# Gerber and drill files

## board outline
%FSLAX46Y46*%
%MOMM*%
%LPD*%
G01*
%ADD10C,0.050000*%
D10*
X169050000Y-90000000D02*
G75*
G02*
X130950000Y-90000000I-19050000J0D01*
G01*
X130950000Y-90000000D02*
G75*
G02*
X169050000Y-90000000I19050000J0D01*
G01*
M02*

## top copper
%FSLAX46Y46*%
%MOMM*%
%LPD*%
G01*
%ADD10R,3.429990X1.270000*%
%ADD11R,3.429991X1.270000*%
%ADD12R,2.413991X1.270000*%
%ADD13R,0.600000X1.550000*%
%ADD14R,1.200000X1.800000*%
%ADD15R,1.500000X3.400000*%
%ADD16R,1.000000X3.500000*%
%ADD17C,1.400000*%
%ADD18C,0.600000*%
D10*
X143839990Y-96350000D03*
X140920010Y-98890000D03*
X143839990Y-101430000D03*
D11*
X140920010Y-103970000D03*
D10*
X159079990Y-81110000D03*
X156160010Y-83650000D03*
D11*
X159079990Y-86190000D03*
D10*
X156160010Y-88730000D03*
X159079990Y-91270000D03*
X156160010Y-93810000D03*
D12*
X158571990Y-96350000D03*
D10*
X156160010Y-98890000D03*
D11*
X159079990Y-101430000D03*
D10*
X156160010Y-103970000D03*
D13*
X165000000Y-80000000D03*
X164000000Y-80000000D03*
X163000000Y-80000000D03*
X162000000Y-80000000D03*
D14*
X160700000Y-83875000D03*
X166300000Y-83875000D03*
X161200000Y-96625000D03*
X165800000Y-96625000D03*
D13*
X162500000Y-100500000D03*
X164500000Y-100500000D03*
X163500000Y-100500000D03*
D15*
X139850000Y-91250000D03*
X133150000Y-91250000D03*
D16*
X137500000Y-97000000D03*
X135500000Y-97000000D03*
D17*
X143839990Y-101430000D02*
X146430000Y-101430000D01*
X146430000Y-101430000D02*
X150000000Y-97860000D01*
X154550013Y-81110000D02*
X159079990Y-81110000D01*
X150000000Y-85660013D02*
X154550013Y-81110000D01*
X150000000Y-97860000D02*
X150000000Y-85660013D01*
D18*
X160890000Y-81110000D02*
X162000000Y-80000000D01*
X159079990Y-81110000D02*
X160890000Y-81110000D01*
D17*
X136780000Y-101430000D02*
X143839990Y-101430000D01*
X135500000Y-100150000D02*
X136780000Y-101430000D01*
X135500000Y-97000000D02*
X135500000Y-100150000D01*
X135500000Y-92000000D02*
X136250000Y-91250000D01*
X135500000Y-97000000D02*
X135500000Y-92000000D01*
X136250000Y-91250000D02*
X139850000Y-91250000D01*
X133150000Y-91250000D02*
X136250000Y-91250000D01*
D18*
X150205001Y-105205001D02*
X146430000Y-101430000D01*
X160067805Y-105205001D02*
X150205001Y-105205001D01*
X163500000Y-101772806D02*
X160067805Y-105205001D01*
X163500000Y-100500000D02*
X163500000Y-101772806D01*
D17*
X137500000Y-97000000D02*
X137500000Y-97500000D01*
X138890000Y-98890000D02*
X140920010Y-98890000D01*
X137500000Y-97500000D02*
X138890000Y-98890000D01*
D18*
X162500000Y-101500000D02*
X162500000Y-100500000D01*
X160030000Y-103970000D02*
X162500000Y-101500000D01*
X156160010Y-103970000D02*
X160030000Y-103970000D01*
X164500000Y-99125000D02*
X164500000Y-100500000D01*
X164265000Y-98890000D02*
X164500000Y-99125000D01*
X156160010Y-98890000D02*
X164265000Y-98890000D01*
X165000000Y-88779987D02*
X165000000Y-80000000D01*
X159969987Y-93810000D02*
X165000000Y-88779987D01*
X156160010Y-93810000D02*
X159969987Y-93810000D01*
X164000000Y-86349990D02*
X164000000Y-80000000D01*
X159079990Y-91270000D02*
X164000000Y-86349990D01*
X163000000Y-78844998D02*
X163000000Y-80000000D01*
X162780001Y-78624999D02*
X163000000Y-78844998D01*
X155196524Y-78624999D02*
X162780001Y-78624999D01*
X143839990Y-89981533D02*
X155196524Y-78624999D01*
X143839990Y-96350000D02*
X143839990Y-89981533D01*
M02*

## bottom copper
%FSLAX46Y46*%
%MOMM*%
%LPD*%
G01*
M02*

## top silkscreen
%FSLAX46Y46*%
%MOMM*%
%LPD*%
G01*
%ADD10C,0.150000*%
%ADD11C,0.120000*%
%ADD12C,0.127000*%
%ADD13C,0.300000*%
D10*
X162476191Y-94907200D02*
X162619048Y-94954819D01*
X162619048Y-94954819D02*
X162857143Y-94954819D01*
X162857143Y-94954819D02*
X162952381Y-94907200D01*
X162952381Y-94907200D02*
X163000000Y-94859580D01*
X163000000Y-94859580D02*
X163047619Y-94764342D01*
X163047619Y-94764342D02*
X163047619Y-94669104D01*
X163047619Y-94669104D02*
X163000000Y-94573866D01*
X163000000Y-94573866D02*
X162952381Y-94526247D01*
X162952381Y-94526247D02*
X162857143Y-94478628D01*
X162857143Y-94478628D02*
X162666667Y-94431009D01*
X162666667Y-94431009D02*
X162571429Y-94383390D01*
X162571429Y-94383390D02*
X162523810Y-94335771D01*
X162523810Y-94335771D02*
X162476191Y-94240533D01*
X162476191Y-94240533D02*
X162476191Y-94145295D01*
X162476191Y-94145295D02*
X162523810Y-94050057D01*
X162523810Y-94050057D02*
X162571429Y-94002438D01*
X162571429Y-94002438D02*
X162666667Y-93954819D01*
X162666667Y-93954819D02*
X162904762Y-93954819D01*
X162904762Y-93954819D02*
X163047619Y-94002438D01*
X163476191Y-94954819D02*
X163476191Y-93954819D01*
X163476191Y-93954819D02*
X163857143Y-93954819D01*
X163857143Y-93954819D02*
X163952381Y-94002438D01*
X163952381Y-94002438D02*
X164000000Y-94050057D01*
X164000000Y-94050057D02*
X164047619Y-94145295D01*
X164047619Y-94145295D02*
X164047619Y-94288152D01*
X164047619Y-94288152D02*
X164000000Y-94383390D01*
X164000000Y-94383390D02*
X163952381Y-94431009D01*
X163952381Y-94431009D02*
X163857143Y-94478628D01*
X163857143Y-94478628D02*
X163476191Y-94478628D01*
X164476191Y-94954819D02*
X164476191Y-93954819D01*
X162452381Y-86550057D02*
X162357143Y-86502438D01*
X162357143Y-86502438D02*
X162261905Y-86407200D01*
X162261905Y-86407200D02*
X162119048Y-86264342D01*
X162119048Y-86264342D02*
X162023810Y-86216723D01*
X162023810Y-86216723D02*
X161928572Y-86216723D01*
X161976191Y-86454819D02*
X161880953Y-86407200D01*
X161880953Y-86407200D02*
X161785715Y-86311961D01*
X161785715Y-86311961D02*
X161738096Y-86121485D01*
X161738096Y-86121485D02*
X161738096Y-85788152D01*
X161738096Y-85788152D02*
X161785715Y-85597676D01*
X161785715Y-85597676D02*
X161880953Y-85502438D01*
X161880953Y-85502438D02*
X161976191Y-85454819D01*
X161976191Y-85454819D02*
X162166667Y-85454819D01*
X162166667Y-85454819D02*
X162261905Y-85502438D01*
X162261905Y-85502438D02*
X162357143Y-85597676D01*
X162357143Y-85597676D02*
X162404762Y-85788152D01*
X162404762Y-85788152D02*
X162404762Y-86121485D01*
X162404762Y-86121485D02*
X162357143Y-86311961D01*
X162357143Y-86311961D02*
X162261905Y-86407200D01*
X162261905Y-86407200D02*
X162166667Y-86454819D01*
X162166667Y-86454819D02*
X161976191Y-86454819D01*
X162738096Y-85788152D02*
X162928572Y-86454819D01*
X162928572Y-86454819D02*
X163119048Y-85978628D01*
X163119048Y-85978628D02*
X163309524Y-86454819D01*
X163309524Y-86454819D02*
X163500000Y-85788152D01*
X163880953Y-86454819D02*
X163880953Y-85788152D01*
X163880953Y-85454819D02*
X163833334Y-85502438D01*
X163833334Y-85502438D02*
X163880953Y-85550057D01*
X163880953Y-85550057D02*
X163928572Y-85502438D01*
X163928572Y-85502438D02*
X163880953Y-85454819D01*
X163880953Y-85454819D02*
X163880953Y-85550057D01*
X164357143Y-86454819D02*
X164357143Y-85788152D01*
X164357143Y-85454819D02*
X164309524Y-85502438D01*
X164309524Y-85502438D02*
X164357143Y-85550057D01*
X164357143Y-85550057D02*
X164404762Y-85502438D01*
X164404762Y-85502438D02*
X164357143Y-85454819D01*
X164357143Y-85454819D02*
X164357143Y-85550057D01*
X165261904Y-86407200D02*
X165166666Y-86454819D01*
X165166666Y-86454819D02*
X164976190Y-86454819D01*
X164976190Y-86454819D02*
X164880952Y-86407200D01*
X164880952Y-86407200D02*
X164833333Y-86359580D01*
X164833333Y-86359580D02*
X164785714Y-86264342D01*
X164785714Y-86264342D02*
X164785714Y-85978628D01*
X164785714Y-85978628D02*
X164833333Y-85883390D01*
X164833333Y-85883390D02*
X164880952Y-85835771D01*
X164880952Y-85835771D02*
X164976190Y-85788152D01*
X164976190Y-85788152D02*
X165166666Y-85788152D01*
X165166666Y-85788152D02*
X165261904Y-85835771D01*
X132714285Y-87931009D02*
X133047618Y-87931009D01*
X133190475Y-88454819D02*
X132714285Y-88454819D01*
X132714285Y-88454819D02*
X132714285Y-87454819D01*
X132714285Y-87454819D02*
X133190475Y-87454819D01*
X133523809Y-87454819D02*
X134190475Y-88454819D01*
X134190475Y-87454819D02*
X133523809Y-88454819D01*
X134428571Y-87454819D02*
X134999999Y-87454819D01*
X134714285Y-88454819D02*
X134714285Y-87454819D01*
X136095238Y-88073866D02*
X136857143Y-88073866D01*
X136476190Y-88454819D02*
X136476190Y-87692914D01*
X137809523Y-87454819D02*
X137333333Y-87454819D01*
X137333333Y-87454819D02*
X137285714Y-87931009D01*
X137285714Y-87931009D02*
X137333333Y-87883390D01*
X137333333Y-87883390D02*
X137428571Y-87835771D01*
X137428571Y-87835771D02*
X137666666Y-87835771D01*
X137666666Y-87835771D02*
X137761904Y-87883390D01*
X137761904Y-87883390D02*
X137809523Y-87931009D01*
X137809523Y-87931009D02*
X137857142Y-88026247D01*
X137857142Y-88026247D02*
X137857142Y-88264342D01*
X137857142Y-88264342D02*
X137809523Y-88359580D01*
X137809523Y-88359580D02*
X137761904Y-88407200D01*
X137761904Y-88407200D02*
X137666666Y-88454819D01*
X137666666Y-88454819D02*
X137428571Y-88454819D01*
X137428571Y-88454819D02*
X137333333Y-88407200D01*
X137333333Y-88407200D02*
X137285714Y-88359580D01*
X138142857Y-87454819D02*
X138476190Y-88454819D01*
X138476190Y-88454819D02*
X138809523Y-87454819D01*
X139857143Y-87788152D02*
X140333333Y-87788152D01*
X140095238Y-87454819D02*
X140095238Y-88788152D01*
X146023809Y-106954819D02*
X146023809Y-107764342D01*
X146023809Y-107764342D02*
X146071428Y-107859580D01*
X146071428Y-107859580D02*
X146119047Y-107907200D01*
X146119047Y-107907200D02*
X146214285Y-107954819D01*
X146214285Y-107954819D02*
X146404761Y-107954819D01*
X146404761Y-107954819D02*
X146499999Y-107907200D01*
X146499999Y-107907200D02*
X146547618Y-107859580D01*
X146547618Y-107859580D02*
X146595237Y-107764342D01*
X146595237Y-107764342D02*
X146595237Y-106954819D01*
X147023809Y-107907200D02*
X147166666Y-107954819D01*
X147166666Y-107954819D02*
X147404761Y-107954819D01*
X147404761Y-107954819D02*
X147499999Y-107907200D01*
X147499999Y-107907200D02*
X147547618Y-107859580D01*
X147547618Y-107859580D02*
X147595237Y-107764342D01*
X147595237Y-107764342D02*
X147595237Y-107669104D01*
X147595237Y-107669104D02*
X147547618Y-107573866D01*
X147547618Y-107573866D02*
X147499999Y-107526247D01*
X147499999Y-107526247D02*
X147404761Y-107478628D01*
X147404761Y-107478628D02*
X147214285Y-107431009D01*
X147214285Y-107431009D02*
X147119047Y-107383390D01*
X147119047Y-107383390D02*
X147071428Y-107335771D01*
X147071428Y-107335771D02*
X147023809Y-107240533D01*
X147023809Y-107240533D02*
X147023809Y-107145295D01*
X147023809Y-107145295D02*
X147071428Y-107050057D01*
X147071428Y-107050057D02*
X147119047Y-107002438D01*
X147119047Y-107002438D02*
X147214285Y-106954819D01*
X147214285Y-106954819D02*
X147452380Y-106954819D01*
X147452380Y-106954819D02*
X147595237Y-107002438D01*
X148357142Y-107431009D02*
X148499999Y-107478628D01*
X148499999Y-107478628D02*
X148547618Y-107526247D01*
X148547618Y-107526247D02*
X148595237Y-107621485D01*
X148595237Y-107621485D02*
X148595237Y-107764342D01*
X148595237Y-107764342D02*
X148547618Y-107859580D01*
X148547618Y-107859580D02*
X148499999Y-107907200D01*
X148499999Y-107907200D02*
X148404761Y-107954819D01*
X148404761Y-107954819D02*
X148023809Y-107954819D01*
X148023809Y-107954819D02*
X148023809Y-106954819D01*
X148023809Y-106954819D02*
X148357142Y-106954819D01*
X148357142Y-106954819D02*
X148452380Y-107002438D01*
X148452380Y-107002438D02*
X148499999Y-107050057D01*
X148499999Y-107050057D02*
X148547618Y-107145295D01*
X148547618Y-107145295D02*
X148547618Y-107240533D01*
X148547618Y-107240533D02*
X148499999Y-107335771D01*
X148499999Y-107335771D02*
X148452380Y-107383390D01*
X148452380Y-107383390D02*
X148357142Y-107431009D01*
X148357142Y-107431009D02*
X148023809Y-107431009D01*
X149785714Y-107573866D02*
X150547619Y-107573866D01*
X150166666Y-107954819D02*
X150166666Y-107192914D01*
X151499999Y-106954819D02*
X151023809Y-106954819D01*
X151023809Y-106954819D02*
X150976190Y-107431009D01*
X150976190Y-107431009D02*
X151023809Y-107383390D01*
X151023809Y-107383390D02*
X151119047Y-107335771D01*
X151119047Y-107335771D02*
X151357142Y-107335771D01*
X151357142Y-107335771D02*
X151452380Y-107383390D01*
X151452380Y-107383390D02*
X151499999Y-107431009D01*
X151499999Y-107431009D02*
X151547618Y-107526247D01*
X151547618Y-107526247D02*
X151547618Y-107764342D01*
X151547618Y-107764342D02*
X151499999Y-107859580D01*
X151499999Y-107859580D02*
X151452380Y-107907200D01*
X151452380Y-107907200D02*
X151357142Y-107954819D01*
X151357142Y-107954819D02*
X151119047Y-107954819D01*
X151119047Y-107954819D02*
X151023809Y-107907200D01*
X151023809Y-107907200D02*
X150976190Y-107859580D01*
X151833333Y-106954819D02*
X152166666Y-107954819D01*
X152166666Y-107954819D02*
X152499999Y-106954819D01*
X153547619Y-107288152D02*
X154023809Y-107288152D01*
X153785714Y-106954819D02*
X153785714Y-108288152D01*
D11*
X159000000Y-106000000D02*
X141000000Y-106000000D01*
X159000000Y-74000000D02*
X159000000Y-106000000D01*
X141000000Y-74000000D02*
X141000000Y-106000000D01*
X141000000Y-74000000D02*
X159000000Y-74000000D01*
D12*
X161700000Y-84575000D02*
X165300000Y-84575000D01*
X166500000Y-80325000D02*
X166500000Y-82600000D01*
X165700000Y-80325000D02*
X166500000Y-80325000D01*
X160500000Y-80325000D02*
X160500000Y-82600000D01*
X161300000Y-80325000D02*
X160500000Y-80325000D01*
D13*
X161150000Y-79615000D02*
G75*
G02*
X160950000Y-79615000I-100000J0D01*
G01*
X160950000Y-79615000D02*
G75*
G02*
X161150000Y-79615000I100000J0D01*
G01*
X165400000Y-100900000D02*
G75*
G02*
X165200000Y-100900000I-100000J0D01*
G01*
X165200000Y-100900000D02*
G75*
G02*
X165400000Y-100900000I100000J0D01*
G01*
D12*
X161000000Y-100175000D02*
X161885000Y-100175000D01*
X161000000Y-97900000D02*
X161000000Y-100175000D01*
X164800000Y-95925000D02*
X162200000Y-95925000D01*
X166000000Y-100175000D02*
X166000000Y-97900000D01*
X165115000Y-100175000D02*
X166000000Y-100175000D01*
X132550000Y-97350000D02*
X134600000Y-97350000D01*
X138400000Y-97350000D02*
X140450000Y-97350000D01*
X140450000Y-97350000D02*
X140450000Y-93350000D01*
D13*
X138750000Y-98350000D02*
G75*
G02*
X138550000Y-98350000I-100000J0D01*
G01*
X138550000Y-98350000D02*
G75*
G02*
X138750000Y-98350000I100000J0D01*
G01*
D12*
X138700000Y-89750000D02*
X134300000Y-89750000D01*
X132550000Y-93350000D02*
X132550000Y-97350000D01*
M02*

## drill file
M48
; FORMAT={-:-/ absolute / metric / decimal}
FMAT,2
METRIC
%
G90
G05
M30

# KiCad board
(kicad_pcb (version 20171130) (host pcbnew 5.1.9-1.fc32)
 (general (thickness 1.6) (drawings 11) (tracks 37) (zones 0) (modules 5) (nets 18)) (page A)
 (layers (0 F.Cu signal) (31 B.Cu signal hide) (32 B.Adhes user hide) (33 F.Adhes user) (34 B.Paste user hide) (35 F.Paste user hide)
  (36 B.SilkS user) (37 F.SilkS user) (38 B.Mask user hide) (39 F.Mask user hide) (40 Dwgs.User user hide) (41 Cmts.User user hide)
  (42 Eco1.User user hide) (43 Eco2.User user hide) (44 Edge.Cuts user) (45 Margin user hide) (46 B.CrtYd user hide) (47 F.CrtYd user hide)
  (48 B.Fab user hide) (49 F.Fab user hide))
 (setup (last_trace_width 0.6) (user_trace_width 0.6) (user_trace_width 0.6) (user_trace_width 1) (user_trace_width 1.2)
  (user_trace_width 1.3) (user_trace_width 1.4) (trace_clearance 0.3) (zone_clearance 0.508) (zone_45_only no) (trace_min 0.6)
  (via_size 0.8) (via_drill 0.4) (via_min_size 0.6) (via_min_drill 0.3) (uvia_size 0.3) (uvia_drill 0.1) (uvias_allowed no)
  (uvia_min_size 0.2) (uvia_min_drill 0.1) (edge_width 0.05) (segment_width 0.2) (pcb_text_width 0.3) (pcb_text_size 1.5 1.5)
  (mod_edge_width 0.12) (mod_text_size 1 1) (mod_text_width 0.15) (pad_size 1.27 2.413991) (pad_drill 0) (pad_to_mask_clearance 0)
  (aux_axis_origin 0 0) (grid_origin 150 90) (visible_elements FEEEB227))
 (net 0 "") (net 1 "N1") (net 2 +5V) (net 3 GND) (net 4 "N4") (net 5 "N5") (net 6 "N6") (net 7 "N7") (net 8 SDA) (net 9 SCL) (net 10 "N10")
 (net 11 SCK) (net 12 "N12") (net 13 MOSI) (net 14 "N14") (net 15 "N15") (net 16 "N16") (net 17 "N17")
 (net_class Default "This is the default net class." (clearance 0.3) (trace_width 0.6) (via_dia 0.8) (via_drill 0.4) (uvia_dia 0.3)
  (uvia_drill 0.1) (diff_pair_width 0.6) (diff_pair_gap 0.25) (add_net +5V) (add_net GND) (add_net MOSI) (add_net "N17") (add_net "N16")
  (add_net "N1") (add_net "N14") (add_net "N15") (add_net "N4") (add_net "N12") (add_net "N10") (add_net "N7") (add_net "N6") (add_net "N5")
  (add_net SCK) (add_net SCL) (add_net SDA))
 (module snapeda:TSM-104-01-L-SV (layer F.Cu) (at 142.38 100.16 90)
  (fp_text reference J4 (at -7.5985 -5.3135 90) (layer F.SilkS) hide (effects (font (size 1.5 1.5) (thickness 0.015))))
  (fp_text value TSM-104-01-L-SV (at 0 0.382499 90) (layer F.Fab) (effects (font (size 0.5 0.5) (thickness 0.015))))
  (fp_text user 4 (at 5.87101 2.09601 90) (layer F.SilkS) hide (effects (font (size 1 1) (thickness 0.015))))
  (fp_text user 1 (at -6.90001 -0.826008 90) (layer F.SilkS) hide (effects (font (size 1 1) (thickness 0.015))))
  (pad 4 smd rect (at 3.81 1.45999 90) (size 1.27 3.42999) (layers F.Cu F.Paste) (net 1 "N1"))
  (pad 3 smd rect (at 1.27 -1.45999 90) (size 1.27 3.42999) (layers F.Cu F.Paste) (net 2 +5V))
  (pad 2 smd rect (at -1.27 1.45999 90) (size 1.27 3.42999) (layers F.Cu F.Paste) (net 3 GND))
  (pad 1 smd rect (at -3.81 -1.45999 90) (size 1.27 3.429991) (layers F.Cu F.Paste) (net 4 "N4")))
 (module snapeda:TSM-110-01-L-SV (layer F.Cu) (at 157.62 92.54 90)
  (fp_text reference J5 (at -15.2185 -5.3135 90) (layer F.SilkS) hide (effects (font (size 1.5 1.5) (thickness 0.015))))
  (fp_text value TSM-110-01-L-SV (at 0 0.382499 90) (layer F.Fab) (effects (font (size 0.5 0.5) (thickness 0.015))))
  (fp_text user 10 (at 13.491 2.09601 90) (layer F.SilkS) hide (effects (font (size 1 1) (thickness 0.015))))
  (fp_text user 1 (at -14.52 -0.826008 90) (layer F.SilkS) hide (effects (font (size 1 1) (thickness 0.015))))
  (pad 10 smd rect (at 11.43 1.45999 90) (size 1.27 3.42999) (layers F.Cu F.Paste) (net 3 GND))
  (pad 9 smd rect (at 8.89 -1.45999 90) (size 1.27 3.42999) (layers F.Cu F.Paste) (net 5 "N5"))
  (pad 8 smd rect (at 6.35 1.45999 90) (size 1.27 3.429991) (layers F.Cu F.Paste) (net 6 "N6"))
  (pad 7 smd rect (at 3.81 -1.45999 90) (size 1.27 3.42999) (layers F.Cu F.Paste) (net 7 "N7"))
  (pad 6 smd rect (at 1.27 1.45999 90) (size 1.27 3.42999) (layers F.Cu F.Paste) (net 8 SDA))
  (pad 5 smd rect (at -1.27 -1.45999 90) (size 1.27 3.42999) (layers F.Cu F.Paste) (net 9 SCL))
  (pad 4 smd rect (at -3.81 0.95199 90) (size 1.27 2.413991) (layers F.Cu F.Paste) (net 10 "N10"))
  (pad 3 smd rect (at -6.35 -1.45999 90) (size 1.27 3.42999) (layers F.Cu F.Paste) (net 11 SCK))
  (pad 2 smd rect (at -8.89 1.45999 90) (size 1.27 3.429991) (layers F.Cu F.Paste) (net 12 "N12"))
  (pad 1 smd rect (at -11.43 -1.45999 90) (size 1.27 3.42999) (layers F.Cu F.Paste) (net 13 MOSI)))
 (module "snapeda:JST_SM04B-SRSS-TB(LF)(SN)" (layer F.Cu) (at 163.5 80)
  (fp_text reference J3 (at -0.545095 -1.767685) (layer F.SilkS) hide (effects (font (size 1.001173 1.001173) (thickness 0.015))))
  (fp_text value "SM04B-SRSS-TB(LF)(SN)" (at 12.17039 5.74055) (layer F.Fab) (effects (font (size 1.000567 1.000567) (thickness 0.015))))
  (fp_line (start -1.8 4.575) (end 1.8 4.575) (layer F.SilkS) (width 0.127))
  (fp_line (start 3 0.325) (end 3 2.6) (layer F.SilkS) (width 0.127))
  (fp_line (start 2.2 0.325) (end 3 0.325) (layer F.SilkS) (width 0.127))
  (fp_line (start -3 0.325) (end -3 2.6) (layer F.SilkS) (width 0.127))
  (fp_line (start -2.2 0.325) (end -3 0.325) (layer F.SilkS) (width 0.127))
  (fp_circle (center -2.45 -0.385) (end -2.35 -0.385) (layer F.SilkS) (width 0.3))
  (pad 4 smd rect (at 1.5 0) (size 0.6 1.55) (layers F.Cu F.Paste F.Mask) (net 9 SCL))
  (pad 3 smd rect (at 0.5 0) (size 0.6 1.55) (layers F.Cu F.Paste F.Mask) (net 8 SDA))
  (pad 2 smd rect (at -0.5 0) (size 0.6 1.55) (layers F.Cu F.Paste F.Mask) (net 1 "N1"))
  (pad 1 smd rect (at -1.5 0) (size 0.6 1.55) (layers F.Cu F.Paste F.Mask) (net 3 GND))
  (pad S1 smd rect (at -2.8 3.875) (size 1.2 1.8) (layers F.Cu F.Paste F.Mask) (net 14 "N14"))
  (pad S2 smd rect (at 2.8 3.875) (size 1.2 1.8) (layers F.Cu F.Paste F.Mask) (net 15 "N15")))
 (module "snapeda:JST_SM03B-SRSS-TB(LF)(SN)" (layer F.Cu) (at 163.5 100.5 180)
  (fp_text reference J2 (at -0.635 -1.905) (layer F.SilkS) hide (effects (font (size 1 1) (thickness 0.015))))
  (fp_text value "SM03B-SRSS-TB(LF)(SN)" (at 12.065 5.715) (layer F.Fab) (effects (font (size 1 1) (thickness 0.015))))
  (fp_circle (center -1.8 -0.4) (end -1.7 -0.4) (layer F.SilkS) (width 0.3))
  (fp_line (start 2.5 0.325) (end 1.615 0.325) (layer F.SilkS) (width 0.127))
  (fp_line (start 2.5 2.6) (end 2.5 0.325) (layer F.SilkS) (width 0.127))
  (fp_line (start -1.3 4.575) (end 1.3 4.575) (layer F.SilkS) (width 0.127))
  (fp_line (start -2.5 0.325) (end -2.5 2.6) (layer F.SilkS) (width 0.127))
  (fp_line (start -1.615 0.325) (end -2.5 0.325) (layer F.SilkS) (width 0.127))
  (pad S2 smd rect (at 2.3 3.875 180) (size 1.2 1.8) (layers F.Cu F.Paste F.Mask) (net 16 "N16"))
  (pad S1 smd rect (at -2.3 3.875 180) (size 1.2 1.8) (layers F.Cu F.Paste F.Mask) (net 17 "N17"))
  (pad 3 smd rect (at 1 0 180) (size 0.6 1.55) (layers F.Cu F.Paste F.Mask) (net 13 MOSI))
  (pad 1 smd rect (at -1 0 180) (size 0.6 1.55) (layers F.Cu F.Paste F.Mask) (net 11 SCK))
  (pad 2 smd rect (at 0 0 180) (size 0.6 1.55) (layers F.Cu F.Paste F.Mask) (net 3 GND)))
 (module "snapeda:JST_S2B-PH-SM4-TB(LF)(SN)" (layer F.Cu) (at 136.5 97 180)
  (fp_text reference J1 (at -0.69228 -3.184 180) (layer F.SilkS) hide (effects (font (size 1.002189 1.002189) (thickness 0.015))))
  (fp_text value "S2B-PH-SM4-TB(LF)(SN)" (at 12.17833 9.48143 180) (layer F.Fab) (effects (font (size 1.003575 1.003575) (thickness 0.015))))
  (fp_line (start 3.95 -0.35) (end 1.9 -0.35) (layer F.SilkS) (width 0.127))
  (fp_line (start -1.9 -0.35) (end -3.95 -0.35) (layer F.SilkS) (width 0.127))
  (fp_line (start -3.95 -0.35) (end -3.95 3.65) (layer F.SilkS) (width 0.127))
  (fp_circle (center -2.15 -1.35) (end -2.05 -1.35) (layer F.SilkS) (width 0.3))
  (fp_line (start -2.2 7.25) (end 2.2 7.25) (layer F.SilkS) (width 0.127))
  (fp_line (start 3.95 3.65) (end 3.95 -0.35) (layer F.SilkS) (width 0.127))
  (pad S1 smd rect (at -3.35 5.75 180) (size 1.5 3.4) (layers F.Cu F.Paste F.Mask) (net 3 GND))
  (pad S2 smd rect (at 3.35 5.75 180) (size 1.5 3.4) (layers F.Cu F.Paste F.Mask) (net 3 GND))
  (pad 1 smd rect (at -1 0 180) (size 1 3.5) (layers F.Cu F.Paste F.Mask) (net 2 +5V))
  (pad 2 smd rect (at 1 0 180) (size 1 3.5) (layers F.Cu F.Paste F.Mask) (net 3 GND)))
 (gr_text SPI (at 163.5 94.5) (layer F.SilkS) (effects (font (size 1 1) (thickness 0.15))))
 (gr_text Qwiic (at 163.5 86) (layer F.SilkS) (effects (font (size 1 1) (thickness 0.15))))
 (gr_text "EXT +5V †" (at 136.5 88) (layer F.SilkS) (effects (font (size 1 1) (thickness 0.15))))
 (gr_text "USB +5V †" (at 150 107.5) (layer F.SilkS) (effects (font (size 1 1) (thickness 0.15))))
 (gr_circle (center 150 90) (end 169.05 90) (layer Edge.Cuts) (width 0.05))
 (gr_line (start 159 106) (end 141 106) (layer F.SilkS) (width 0.12))
 (gr_line (start 159 74) (end 159 106) (layer F.SilkS) (width 0.12))
 (gr_line (start 141 74) (end 141 106) (layer F.SilkS) (width 0.12))
 (gr_line (start 141 74) (end 159 74) (layer F.SilkS) (width 0.12))
 (segment (start 143.83999 101.43) (end 146.43 101.43) (width 1.4) (layer F.Cu) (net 3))
 (segment (start 146.43 101.43) (end 150 97.86) (width 1.4) (layer F.Cu) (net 3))
 (segment (start 154.550013 81.11) (end 159.07999 81.11) (width 1.4) (layer F.Cu) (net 3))
 (segment (start 150 85.660013) (end 154.550013 81.11) (width 1.4) (layer F.Cu) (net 3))
 (segment (start 150 97.86) (end 150 85.660013) (width 1.4) (layer F.Cu) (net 3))
 (segment (start 160.89 81.11) (end 162 80) (width 0.6) (layer F.Cu) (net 3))
 (segment (start 159.07999 81.11) (end 160.89 81.11) (width 0.6) (layer F.Cu) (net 3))
 (segment (start 136.78 101.43) (end 143.83999 101.43) (width 1.4) (layer F.Cu) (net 3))
 (segment (start 135.5 100.15) (end 136.78 101.43) (width 1.4) (layer F.Cu) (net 3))
 (segment (start 135.5 97) (end 135.5 100.15) (width 1.4) (layer F.Cu) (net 3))
 (segment (start 135.5 92) (end 136.25 91.25) (width 1.4) (layer F.Cu) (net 3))
 (segment (start 135.5 97) (end 135.5 92) (width 1.4) (layer F.Cu) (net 3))
 (segment (start 136.25 91.25) (end 139.85 91.25) (width 1.4) (layer F.Cu) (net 3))
 (segment (start 133.15 91.25) (end 136.25 91.25) (width 1.4) (layer F.Cu) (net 3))
 (segment (start 150.205001 105.205001) (end 146.43 101.43) (width 0.6) (layer F.Cu) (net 3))
 (segment (start 160.067805 105.205001) (end 150.205001 105.205001) (width 0.6) (layer F.Cu) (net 3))
 (segment (start 163.5 101.772806) (end 160.067805 105.205001) (width 0.6) (layer F.Cu) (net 3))
 (segment (start 163.5 100.5) (end 163.5 101.772806) (width 0.6) (layer F.Cu) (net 3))
 (segment (start 137.5 97) (end 137.5 97.5) (width 1.4) (layer F.Cu) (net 2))
 (segment (start 138.89 98.89) (end 140.92001 98.89) (width 1.4) (layer F.Cu) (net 2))
 (segment (start 137.5 97.5) (end 138.89 98.89) (width 1.4) (layer F.Cu) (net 2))
 (segment (start 162.5 101.5) (end 162.5 100.5) (width 0.6) (layer F.Cu) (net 13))
 (segment (start 160.03 103.97) (end 162.5 101.5) (width 0.6) (layer F.Cu) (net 13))
 (segment (start 156.16001 103.97) (end 160.03 103.97) (width 0.6) (layer F.Cu) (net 13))
 (segment (start 164.5 99.125) (end 164.5 100.5) (width 0.6) (layer F.Cu) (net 11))
 (segment (start 164.265 98.89) (end 164.5 99.125) (width 0.6) (layer F.Cu) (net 11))
 (segment (start 156.16001 98.89) (end 164.265 98.89) (width 0.6) (layer F.Cu) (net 11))
 (segment (start 165 88.779987) (end 165 80) (width 0.6) (layer F.Cu) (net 9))
 (segment (start 159.969987 93.81) (end 165 88.779987) (width 0.6) (layer F.Cu) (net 9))
 (segment (start 156.16001 93.81) (end 159.969987 93.81) (width 0.6) (layer F.Cu) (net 9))
 (segment (start 164 86.34999) (end 164 80) (width 0.6) (layer F.Cu) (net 8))
 (segment (start 159.07999 91.27) (end 164 86.34999) (width 0.6) (layer F.Cu) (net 8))
 (segment (start 163 78.844998) (end 163 80) (width 0.6) (layer F.Cu) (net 1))
 (segment (start 162.780001 78.624999) (end 163 78.844998) (width 0.6) (layer F.Cu) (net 1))
 (segment (start 155.196524 78.624999) (end 162.780001 78.624999) (width 0.6) (layer F.Cu) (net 1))
 (segment (start 143.83999 89.981533) (end 155.196524 78.624999) (width 0.6) (layer F.Cu) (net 1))
 (segment (start 143.83999 96.35) (end 143.83999 89.981533) (width 0.6) (layer F.Cu) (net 1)))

